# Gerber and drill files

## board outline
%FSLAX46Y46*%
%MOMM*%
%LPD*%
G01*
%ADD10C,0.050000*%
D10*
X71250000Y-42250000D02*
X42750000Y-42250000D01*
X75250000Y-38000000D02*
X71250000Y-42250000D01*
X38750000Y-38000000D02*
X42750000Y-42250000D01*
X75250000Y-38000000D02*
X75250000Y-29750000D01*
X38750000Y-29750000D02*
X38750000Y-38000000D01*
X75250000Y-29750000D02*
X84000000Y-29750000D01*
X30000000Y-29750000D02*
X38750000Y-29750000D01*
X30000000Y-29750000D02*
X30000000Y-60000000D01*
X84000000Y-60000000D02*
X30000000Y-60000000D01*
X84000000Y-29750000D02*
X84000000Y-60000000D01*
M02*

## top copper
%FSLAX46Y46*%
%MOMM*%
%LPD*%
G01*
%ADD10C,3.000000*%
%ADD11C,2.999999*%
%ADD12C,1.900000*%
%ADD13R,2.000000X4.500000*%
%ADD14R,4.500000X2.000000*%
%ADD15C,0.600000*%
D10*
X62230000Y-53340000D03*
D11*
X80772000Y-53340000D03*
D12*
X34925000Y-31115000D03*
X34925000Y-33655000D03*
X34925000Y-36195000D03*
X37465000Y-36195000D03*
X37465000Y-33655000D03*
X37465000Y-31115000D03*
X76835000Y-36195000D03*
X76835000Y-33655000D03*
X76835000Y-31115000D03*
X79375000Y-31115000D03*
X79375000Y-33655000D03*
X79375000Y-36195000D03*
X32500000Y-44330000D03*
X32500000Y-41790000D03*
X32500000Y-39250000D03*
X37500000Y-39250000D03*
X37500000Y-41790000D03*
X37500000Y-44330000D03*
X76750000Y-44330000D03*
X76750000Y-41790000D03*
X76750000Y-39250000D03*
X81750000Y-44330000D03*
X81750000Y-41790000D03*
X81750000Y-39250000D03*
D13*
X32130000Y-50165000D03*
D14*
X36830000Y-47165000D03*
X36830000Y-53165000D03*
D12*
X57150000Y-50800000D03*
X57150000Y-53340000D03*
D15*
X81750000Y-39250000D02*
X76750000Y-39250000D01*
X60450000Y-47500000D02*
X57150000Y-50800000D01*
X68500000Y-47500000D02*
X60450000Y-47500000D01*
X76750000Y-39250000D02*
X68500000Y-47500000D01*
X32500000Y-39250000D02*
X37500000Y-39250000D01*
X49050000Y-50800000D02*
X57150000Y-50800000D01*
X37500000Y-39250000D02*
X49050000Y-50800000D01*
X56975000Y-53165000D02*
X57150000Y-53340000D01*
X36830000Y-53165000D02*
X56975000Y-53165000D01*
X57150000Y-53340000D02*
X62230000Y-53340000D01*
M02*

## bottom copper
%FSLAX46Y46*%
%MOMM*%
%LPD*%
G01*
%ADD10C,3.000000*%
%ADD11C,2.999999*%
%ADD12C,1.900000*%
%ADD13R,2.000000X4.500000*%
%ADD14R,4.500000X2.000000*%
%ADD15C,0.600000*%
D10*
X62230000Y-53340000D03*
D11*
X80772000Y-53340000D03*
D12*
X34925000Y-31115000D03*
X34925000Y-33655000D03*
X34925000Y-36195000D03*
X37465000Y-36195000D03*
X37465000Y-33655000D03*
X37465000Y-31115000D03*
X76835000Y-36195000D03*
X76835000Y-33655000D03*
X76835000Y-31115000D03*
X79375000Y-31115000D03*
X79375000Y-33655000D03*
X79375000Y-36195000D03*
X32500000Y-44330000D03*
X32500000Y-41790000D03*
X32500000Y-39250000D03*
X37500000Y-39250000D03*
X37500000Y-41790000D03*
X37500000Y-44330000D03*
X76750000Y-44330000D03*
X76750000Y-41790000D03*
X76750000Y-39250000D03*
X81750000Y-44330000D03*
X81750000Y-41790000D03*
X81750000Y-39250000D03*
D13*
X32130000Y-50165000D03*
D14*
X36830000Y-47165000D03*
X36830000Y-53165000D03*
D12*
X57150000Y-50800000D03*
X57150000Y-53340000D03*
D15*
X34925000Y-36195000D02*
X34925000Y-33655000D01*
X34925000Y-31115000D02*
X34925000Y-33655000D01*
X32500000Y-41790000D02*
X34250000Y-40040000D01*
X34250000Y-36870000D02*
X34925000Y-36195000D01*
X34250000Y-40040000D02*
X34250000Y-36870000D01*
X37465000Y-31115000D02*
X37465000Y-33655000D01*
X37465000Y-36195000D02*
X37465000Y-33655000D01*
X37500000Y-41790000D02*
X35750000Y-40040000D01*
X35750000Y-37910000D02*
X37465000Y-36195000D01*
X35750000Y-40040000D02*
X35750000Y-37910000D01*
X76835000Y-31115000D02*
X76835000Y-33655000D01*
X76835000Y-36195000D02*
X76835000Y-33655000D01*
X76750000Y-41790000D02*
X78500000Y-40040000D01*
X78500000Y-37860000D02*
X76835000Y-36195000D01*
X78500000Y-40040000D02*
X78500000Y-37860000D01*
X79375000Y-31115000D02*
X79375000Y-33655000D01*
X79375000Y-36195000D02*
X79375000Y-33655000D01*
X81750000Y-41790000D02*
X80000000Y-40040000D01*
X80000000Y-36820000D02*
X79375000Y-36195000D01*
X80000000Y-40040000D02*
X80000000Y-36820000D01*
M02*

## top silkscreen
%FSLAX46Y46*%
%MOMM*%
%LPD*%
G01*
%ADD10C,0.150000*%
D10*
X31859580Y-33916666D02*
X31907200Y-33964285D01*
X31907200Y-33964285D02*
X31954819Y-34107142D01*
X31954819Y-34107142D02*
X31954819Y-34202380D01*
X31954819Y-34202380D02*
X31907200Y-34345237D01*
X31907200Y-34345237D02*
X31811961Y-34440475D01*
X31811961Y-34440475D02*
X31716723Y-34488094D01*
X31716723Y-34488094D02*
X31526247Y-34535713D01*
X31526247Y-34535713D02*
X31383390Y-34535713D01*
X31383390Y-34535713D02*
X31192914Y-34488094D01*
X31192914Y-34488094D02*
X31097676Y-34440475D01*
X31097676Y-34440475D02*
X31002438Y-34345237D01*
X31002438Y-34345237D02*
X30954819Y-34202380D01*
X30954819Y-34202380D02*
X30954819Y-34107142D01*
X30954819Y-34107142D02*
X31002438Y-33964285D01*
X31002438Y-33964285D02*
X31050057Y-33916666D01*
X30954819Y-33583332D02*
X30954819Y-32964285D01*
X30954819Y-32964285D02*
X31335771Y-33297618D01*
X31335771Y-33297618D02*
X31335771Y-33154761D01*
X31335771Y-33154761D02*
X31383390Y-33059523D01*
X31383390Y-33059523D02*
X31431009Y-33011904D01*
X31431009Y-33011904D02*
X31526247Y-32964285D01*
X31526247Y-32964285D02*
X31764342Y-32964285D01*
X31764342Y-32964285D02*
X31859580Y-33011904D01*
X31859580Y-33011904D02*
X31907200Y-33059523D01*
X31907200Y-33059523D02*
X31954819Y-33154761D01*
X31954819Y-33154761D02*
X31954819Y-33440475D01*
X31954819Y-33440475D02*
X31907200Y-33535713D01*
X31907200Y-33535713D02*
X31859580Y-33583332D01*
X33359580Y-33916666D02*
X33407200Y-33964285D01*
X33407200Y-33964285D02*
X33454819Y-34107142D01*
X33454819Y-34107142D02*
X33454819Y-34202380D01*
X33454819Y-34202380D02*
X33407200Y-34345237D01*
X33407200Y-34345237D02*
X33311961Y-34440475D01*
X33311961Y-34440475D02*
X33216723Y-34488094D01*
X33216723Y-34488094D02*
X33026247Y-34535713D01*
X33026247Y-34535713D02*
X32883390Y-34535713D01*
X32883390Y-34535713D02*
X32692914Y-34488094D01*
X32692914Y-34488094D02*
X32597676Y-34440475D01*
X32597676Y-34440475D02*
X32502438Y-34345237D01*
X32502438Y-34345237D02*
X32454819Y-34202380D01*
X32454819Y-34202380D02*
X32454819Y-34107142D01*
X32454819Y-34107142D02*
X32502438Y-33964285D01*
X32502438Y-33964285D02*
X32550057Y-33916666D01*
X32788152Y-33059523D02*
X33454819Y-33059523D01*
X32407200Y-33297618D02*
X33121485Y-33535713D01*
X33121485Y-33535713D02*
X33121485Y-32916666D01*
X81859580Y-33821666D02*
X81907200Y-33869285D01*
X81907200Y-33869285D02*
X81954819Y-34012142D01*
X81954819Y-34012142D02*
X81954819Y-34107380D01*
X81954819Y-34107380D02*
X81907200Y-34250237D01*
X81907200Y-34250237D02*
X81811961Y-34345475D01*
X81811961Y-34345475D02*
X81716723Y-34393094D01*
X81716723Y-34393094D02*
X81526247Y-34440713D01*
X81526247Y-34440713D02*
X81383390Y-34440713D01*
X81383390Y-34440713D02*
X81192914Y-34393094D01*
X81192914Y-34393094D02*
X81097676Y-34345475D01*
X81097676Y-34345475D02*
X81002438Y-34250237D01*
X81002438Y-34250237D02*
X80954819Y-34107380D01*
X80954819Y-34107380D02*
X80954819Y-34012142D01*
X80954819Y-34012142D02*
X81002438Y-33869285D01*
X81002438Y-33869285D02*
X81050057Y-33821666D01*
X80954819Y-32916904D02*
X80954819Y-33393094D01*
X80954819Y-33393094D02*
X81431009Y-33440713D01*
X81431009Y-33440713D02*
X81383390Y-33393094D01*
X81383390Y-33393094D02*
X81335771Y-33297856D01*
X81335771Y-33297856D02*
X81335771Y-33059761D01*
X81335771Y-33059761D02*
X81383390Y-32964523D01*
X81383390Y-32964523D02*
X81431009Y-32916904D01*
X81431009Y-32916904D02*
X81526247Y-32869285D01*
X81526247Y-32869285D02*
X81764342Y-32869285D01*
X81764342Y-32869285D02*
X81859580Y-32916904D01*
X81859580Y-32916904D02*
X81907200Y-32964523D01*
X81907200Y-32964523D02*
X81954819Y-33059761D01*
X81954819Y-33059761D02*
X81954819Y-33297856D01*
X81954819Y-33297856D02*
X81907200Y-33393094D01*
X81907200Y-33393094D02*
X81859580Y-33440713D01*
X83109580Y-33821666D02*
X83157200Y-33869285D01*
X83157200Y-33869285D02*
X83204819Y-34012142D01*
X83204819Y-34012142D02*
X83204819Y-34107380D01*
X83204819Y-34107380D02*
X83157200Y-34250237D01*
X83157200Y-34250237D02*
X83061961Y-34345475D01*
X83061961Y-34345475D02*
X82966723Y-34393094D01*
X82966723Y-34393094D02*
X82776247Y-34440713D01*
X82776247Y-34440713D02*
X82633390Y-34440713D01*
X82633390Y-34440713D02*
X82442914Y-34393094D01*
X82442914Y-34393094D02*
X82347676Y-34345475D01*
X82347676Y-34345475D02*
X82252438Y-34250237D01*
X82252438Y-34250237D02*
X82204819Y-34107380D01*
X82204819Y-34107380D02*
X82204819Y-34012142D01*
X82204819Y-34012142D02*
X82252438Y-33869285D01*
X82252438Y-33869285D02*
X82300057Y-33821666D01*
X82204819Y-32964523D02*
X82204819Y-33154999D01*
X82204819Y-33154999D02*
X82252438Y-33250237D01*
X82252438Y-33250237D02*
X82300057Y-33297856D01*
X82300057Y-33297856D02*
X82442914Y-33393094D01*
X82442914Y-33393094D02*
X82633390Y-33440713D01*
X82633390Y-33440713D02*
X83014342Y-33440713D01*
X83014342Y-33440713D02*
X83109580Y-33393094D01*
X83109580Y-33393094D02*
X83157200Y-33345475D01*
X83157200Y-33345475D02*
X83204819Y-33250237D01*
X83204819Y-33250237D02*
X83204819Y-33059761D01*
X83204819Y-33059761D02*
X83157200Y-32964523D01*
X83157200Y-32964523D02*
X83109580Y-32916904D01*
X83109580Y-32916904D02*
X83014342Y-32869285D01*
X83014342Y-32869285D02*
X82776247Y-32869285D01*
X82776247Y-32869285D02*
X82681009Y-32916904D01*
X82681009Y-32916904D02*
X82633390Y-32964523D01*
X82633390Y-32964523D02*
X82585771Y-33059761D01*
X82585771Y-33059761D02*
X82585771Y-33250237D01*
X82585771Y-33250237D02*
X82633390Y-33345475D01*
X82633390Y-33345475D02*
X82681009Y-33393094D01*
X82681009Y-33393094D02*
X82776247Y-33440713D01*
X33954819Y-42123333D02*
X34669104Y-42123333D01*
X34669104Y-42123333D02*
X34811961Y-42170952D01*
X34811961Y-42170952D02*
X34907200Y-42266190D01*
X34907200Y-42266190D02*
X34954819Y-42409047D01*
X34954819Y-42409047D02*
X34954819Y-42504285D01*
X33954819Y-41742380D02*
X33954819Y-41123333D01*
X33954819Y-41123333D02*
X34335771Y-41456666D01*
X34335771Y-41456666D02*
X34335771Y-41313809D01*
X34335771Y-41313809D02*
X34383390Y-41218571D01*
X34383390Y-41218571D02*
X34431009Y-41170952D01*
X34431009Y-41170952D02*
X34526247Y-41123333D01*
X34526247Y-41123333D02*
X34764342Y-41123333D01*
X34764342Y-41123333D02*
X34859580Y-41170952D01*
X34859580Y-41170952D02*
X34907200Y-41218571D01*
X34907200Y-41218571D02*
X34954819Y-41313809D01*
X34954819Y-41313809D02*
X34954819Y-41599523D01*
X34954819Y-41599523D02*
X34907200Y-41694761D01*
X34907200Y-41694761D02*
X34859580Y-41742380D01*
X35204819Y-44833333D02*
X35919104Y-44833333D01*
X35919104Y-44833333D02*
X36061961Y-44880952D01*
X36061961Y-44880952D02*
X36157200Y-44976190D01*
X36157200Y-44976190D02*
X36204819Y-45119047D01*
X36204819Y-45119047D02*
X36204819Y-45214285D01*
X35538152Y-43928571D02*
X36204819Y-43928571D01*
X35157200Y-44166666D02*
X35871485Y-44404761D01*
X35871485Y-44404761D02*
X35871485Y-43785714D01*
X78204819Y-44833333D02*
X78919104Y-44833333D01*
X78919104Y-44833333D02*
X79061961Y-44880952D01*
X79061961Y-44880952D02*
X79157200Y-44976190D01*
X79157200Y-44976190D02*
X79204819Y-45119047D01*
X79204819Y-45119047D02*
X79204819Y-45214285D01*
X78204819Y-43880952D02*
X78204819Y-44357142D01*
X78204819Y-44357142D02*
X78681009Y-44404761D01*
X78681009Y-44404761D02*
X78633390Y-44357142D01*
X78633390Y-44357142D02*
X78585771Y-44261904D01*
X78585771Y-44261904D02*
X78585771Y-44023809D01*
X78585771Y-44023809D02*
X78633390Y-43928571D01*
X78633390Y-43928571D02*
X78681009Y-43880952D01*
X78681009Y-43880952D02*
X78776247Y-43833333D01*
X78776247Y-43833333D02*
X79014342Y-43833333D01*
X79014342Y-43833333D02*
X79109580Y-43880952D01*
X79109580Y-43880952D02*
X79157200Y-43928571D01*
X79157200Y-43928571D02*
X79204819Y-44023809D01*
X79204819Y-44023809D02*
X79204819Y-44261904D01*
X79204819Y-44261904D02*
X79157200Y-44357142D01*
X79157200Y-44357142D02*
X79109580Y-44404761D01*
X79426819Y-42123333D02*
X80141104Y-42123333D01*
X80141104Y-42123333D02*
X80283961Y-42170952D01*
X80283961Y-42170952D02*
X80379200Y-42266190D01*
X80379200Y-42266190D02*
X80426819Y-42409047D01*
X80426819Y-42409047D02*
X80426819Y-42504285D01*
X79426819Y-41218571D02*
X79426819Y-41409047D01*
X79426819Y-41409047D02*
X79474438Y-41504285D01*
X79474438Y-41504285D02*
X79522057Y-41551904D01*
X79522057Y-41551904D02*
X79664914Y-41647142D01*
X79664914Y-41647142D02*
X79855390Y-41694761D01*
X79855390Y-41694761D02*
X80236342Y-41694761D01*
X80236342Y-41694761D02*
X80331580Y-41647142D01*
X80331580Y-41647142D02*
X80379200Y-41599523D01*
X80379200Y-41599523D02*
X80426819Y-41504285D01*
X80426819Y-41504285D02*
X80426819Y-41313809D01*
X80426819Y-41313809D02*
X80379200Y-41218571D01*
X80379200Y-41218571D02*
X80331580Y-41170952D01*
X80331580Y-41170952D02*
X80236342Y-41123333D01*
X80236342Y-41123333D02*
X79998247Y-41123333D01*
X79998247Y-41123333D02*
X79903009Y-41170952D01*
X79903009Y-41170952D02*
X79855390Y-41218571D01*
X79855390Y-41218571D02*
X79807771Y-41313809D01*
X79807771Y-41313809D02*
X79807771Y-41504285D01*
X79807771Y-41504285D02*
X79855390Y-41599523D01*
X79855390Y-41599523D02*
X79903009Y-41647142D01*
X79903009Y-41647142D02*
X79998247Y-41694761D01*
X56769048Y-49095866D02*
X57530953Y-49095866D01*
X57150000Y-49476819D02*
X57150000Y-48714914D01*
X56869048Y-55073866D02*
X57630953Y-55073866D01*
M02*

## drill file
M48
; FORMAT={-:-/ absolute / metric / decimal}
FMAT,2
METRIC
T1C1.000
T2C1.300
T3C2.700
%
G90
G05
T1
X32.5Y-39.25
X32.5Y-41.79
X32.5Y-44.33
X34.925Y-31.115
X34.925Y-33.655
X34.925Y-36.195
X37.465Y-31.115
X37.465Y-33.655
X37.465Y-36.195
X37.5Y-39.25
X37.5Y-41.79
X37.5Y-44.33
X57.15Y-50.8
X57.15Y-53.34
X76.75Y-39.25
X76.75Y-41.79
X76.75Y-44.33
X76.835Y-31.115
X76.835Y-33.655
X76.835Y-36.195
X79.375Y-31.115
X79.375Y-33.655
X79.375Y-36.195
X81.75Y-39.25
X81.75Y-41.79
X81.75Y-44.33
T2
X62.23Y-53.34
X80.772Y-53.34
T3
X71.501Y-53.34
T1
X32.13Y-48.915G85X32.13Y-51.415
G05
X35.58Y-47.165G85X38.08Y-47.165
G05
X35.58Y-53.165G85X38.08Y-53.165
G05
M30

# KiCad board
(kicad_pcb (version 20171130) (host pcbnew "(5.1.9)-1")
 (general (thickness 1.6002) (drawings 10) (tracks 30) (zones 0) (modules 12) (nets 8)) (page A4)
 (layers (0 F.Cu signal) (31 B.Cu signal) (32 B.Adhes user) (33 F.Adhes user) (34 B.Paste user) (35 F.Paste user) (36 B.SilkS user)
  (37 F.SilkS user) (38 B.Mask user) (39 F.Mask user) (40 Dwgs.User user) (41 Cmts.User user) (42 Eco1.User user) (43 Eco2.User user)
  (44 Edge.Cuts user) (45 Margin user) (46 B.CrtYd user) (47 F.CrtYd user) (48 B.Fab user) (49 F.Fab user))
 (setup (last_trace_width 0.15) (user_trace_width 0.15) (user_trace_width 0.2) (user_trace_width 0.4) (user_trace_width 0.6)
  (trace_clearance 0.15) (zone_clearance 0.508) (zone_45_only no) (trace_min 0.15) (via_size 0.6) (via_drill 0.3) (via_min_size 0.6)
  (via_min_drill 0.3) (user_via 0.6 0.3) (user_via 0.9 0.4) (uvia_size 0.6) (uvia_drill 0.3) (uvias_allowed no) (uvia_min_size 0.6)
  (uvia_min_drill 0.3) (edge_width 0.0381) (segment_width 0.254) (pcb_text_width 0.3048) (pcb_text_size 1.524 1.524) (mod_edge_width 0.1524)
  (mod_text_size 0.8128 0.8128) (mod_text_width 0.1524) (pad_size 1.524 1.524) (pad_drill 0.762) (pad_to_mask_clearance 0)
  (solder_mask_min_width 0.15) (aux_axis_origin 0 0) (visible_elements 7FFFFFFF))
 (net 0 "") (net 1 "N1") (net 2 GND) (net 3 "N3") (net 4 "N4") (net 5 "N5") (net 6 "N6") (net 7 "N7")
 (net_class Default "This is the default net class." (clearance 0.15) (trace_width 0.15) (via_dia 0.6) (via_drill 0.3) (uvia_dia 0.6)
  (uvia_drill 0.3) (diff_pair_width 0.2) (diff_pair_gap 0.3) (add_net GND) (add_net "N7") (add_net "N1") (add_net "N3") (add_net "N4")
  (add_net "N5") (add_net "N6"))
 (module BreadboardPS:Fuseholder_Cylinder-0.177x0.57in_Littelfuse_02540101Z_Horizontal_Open (layer B.Cu) (at 62.23 53.34)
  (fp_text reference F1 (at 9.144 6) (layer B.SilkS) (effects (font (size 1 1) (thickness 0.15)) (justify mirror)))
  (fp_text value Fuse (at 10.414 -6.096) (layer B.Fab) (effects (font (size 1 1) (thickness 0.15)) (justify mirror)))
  (pad 1 thru_hole circle (at 0 0) (size 3 3) (drill 1.3) (layers *.Cu *.Mask) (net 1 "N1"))
  (pad 2 thru_hole circle (at 18.542 0) (size 2.999999 2.999999) (drill 1.3) (layers *.Cu *.Mask) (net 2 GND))
  (pad "" np_thru_hole circle (at 9.271 0) (size 2.7 2.7) (drill 2.7) (layers *.Cu *.Mask)))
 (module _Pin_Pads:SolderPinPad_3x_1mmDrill (layer F.Cu) (at 34.925 33.655 90)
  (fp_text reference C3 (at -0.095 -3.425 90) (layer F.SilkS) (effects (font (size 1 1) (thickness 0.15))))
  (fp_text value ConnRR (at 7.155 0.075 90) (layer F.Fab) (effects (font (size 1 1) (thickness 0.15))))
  (pad 1 thru_hole circle (at 2.54 0 90) (size 1.9 1.9) (drill 1) (layers *.Cu *.Mask) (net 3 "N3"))
  (pad 1 thru_hole circle (at 0 0 90) (size 1.9 1.9) (drill 1) (layers *.Cu *.Mask) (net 3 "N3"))
  (pad 1 thru_hole circle (at -2.54 0 90) (size 1.9 1.9) (drill 1) (layers *.Cu *.Mask) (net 3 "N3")))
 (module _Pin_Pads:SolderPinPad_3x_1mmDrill (layer F.Cu) (at 37.465 33.655 90)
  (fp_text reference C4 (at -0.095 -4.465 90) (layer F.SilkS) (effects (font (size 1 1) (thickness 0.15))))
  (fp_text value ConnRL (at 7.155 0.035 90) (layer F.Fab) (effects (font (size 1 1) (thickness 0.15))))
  (pad 1 thru_hole circle (at -2.54 0 90) (size 1.9 1.9) (drill 1) (layers *.Cu *.Mask) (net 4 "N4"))
  (pad 1 thru_hole circle (at 0 0 90) (size 1.9 1.9) (drill 1) (layers *.Cu *.Mask) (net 4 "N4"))
  (pad 1 thru_hole circle (at 2.54 0 90) (size 1.9 1.9) (drill 1) (layers *.Cu *.Mask) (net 4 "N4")))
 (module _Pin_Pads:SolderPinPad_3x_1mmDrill (layer F.Cu) (at 76.835 33.655 90)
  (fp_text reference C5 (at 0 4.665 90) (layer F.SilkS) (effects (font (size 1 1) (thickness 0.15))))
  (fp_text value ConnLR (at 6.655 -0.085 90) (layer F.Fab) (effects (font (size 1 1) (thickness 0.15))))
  (pad 1 thru_hole circle (at -2.54 0 90) (size 1.9 1.9) (drill 1) (layers *.Cu *.Mask) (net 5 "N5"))
  (pad 1 thru_hole circle (at 0 0 90) (size 1.9 1.9) (drill 1) (layers *.Cu *.Mask) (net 5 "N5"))
  (pad 1 thru_hole circle (at 2.54 0 90) (size 1.9 1.9) (drill 1) (layers *.Cu *.Mask) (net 5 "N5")))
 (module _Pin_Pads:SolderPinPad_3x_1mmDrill (layer F.Cu) (at 79.375 33.655 90)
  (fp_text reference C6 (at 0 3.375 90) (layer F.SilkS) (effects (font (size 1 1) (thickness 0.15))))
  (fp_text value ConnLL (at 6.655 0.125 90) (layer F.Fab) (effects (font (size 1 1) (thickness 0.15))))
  (pad 1 thru_hole circle (at 2.54 0 90) (size 1.9 1.9) (drill 1) (layers *.Cu *.Mask) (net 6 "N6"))
  (pad 1 thru_hole circle (at 0 0 90) (size 1.9 1.9) (drill 1) (layers *.Cu *.Mask) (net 6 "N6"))
  (pad 1 thru_hole circle (at -2.54 0 90) (size 1.9 1.9) (drill 1) (layers *.Cu *.Mask) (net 6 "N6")))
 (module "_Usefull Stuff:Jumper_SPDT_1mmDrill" (layer F.Cu) (at 32.5 41.79 90)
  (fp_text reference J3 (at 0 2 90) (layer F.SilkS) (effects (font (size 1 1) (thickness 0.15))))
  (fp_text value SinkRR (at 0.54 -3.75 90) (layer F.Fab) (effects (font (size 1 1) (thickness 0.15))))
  (pad 1 thru_hole circle (at -2.54 0 90) (size 1.9 1.9) (drill 1) (layers *.Cu *.Mask) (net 2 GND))
  (pad 2 thru_hole circle (at 0 0 90) (size 1.9 1.9) (drill 1) (layers *.Cu *.Mask) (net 3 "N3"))
  (pad 3 thru_hole circle (at 2.54 0 90) (size 1.9 1.9) (drill 1) (layers *.Cu *.Mask) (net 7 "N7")))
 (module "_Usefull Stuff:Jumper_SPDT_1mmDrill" (layer F.Cu) (at 37.5 41.79 90)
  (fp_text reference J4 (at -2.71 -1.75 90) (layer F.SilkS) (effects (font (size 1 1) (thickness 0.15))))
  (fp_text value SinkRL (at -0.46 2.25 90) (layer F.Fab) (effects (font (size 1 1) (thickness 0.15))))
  (pad 3 thru_hole circle (at 2.54 0 90) (size 1.9 1.9) (drill 1) (layers *.Cu *.Mask) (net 7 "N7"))
  (pad 2 thru_hole circle (at 0 0 90) (size 1.9 1.9) (drill 1) (layers *.Cu *.Mask) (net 4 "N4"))
  (pad 1 thru_hole circle (at -2.54 0 90) (size 1.9 1.9) (drill 1) (layers *.Cu *.Mask) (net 2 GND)))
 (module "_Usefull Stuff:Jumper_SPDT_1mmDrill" (layer F.Cu) (at 76.75 41.79 90)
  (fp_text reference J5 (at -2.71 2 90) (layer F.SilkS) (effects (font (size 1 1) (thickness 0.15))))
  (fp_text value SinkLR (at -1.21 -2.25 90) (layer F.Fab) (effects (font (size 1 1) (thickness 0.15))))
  (pad 1 thru_hole circle (at -2.54 0 90) (size 1.9 1.9) (drill 1) (layers *.Cu *.Mask) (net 2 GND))
  (pad 2 thru_hole circle (at 0 0 90) (size 1.9 1.9) (drill 1) (layers *.Cu *.Mask) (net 5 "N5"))
  (pad 3 thru_hole circle (at 2.54 0 90) (size 1.9 1.9) (drill 1) (layers *.Cu *.Mask) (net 7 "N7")))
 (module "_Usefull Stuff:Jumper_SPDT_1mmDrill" (layer F.Cu) (at 81.75 41.79 90)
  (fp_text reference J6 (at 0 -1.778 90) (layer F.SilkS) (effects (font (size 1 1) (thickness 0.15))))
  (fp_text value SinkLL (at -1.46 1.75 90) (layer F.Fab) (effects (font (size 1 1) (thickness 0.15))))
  (pad 1 thru_hole circle (at -2.54 0 90) (size 1.9 1.9) (drill 1) (layers *.Cu *.Mask) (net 2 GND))
  (pad 2 thru_hole circle (at 0 0 90) (size 1.9 1.9) (drill 1) (layers *.Cu *.Mask) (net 6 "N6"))
  (pad 3 thru_hole circle (at 2.54 0 90) (size 1.9 1.9) (drill 1) (layers *.Cu *.Mask) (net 7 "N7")))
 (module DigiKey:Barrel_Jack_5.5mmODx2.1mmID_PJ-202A (layer B.Cu) (at 36.83 50.165)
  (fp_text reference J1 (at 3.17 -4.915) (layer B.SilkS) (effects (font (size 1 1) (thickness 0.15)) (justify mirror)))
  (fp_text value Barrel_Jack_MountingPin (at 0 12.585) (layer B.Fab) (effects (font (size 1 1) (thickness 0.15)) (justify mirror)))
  (pad 3 thru_hole rect (at -4.7 0) (size 2 4.5) (drill oval 1 3.5) (layers *.Cu *.Mask))
  (pad 1 thru_hole rect (at 0 -3) (size 4.5 2) (drill oval 3.5 1) (layers *.Cu *.Mask) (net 7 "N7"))
  (pad 2 thru_hole rect (at 0 3) (size 4.5 2) (drill oval 3.5 1) (layers *.Cu *.Mask) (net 1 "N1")))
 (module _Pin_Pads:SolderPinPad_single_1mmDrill (layer F.Cu) (at 57.15 50.8)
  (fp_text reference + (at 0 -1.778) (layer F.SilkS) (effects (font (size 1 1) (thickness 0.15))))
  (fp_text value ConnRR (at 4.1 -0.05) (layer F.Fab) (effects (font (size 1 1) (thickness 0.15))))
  (pad 1 thru_hole circle (at 0 0) (size 1.9 1.9) (drill 1) (layers *.Cu *.Mask) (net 7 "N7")))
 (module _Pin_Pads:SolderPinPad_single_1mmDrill (layer F.Cu) (at 57.15 53.34)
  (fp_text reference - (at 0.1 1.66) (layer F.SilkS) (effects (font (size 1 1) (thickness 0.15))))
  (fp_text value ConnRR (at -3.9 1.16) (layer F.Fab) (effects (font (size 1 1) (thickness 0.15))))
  (pad 1 thru_hole circle (at 0 0) (size 1.9 1.9) (drill 1) (layers *.Cu *.Mask) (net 1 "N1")))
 (gr_line (start 71.25 42.25) (end 42.75 42.25) (layer Edge.Cuts) (width 0.05))
 (gr_line (start 75.25 38) (end 71.25 42.25) (layer Edge.Cuts) (width 0.05))
 (gr_line (start 38.75 38) (end 42.75 42.25) (layer Edge.Cuts) (width 0.05))
 (gr_line (start 75.25 38) (end 75.25 29.75) (layer Edge.Cuts) (width 0.05))
 (gr_line (start 38.75 29.75) (end 38.75 38) (layer Edge.Cuts) (width 0.05))
 (gr_line (start 75.25 29.75) (end 84 29.75) (layer Edge.Cuts) (width 0.05))
 (gr_line (start 30 29.75) (end 38.75 29.75) (layer Edge.Cuts) (width 0.05))
 (gr_line (start 30 29.75) (end 30 60) (layer Edge.Cuts) (width 0.05))
 (gr_line (start 84 60) (end 30 60) (layer Edge.Cuts) (width 0.05))
 (gr_line (start 84 29.75) (end 84 60) (layer Edge.Cuts) (width 0.05))
 (segment (start 34.925 36.195) (end 34.925 33.655) (width 0.6) (layer B.Cu) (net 3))
 (segment (start 34.925 31.115) (end 34.925 33.655) (width 0.6) (layer B.Cu) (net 3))
 (segment (start 32.5 41.79) (end 34.25 40.04) (width 0.6) (layer B.Cu) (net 3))
 (segment (start 34.25 36.87) (end 34.925 36.195) (width 0.6) (layer B.Cu) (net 3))
 (segment (start 34.25 40.04) (end 34.25 36.87) (width 0.6) (layer B.Cu) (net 3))
 (segment (start 37.465 31.115) (end 37.465 33.655) (width 0.6) (layer B.Cu) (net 4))
 (segment (start 37.465 36.195) (end 37.465 33.655) (width 0.6) (layer B.Cu) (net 4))
 (segment (start 37.5 41.79) (end 35.75 40.04) (width 0.6) (layer B.Cu) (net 4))
 (segment (start 35.75 37.91) (end 37.465 36.195) (width 0.6) (layer B.Cu) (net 4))
 (segment (start 35.75 40.04) (end 35.75 37.91) (width 0.6) (layer B.Cu) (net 4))
 (segment (start 76.835 31.115) (end 76.835 33.655) (width 0.6) (layer B.Cu) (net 5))
 (segment (start 76.835 36.195) (end 76.835 33.655) (width 0.6) (layer B.Cu) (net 5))
 (segment (start 76.75 41.79) (end 78.5 40.04) (width 0.6) (layer B.Cu) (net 5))
 (segment (start 78.5 37.86) (end 76.835 36.195) (width 0.6) (layer B.Cu) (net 5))
 (segment (start 78.5 40.04) (end 78.5 37.86) (width 0.6) (layer B.Cu) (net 5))
 (segment (start 79.375 31.115) (end 79.375 33.655) (width 0.6) (layer B.Cu) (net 6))
 (segment (start 79.375 36.195) (end 79.375 33.655) (width 0.6) (layer B.Cu) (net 6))
 (segment (start 81.75 41.79) (end 80 40.04) (width 0.6) (layer B.Cu) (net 6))
 (segment (start 80 36.82) (end 79.375 36.195) (width 0.6) (layer B.Cu) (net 6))
 (segment (start 80 40.04) (end 80 36.82) (width 0.6) (layer B.Cu) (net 6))
 (segment (start 81.75 39.25) (end 76.75 39.25) (width 0.6) (layer F.Cu) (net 7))
 (segment (start 60.45 47.5) (end 57.15 50.8) (width 0.6) (layer F.Cu) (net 7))
 (segment (start 68.5 47.5) (end 60.45 47.5) (width 0.6) (layer F.Cu) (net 7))
 (segment (start 76.75 39.25) (end 68.5 47.5) (width 0.6) (layer F.Cu) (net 7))
 (segment (start 32.5 39.25) (end 37.5 39.25) (width 0.6) (layer F.Cu) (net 7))
 (segment (start 49.05 50.8) (end 57.15 50.8) (width 0.6) (layer F.Cu) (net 7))
 (segment (start 37.5 39.25) (end 49.05 50.8) (width 0.6) (layer F.Cu) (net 7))
 (segment (start 56.975 53.165) (end 57.15 53.34) (width 0.6) (layer F.Cu) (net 1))
 (segment (start 36.83 53.165) (end 56.975 53.165) (width 0.6) (layer F.Cu) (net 1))
 (segment (start 57.15 53.34) (end 62.23 53.34) (width 0.6) (layer F.Cu) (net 1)))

